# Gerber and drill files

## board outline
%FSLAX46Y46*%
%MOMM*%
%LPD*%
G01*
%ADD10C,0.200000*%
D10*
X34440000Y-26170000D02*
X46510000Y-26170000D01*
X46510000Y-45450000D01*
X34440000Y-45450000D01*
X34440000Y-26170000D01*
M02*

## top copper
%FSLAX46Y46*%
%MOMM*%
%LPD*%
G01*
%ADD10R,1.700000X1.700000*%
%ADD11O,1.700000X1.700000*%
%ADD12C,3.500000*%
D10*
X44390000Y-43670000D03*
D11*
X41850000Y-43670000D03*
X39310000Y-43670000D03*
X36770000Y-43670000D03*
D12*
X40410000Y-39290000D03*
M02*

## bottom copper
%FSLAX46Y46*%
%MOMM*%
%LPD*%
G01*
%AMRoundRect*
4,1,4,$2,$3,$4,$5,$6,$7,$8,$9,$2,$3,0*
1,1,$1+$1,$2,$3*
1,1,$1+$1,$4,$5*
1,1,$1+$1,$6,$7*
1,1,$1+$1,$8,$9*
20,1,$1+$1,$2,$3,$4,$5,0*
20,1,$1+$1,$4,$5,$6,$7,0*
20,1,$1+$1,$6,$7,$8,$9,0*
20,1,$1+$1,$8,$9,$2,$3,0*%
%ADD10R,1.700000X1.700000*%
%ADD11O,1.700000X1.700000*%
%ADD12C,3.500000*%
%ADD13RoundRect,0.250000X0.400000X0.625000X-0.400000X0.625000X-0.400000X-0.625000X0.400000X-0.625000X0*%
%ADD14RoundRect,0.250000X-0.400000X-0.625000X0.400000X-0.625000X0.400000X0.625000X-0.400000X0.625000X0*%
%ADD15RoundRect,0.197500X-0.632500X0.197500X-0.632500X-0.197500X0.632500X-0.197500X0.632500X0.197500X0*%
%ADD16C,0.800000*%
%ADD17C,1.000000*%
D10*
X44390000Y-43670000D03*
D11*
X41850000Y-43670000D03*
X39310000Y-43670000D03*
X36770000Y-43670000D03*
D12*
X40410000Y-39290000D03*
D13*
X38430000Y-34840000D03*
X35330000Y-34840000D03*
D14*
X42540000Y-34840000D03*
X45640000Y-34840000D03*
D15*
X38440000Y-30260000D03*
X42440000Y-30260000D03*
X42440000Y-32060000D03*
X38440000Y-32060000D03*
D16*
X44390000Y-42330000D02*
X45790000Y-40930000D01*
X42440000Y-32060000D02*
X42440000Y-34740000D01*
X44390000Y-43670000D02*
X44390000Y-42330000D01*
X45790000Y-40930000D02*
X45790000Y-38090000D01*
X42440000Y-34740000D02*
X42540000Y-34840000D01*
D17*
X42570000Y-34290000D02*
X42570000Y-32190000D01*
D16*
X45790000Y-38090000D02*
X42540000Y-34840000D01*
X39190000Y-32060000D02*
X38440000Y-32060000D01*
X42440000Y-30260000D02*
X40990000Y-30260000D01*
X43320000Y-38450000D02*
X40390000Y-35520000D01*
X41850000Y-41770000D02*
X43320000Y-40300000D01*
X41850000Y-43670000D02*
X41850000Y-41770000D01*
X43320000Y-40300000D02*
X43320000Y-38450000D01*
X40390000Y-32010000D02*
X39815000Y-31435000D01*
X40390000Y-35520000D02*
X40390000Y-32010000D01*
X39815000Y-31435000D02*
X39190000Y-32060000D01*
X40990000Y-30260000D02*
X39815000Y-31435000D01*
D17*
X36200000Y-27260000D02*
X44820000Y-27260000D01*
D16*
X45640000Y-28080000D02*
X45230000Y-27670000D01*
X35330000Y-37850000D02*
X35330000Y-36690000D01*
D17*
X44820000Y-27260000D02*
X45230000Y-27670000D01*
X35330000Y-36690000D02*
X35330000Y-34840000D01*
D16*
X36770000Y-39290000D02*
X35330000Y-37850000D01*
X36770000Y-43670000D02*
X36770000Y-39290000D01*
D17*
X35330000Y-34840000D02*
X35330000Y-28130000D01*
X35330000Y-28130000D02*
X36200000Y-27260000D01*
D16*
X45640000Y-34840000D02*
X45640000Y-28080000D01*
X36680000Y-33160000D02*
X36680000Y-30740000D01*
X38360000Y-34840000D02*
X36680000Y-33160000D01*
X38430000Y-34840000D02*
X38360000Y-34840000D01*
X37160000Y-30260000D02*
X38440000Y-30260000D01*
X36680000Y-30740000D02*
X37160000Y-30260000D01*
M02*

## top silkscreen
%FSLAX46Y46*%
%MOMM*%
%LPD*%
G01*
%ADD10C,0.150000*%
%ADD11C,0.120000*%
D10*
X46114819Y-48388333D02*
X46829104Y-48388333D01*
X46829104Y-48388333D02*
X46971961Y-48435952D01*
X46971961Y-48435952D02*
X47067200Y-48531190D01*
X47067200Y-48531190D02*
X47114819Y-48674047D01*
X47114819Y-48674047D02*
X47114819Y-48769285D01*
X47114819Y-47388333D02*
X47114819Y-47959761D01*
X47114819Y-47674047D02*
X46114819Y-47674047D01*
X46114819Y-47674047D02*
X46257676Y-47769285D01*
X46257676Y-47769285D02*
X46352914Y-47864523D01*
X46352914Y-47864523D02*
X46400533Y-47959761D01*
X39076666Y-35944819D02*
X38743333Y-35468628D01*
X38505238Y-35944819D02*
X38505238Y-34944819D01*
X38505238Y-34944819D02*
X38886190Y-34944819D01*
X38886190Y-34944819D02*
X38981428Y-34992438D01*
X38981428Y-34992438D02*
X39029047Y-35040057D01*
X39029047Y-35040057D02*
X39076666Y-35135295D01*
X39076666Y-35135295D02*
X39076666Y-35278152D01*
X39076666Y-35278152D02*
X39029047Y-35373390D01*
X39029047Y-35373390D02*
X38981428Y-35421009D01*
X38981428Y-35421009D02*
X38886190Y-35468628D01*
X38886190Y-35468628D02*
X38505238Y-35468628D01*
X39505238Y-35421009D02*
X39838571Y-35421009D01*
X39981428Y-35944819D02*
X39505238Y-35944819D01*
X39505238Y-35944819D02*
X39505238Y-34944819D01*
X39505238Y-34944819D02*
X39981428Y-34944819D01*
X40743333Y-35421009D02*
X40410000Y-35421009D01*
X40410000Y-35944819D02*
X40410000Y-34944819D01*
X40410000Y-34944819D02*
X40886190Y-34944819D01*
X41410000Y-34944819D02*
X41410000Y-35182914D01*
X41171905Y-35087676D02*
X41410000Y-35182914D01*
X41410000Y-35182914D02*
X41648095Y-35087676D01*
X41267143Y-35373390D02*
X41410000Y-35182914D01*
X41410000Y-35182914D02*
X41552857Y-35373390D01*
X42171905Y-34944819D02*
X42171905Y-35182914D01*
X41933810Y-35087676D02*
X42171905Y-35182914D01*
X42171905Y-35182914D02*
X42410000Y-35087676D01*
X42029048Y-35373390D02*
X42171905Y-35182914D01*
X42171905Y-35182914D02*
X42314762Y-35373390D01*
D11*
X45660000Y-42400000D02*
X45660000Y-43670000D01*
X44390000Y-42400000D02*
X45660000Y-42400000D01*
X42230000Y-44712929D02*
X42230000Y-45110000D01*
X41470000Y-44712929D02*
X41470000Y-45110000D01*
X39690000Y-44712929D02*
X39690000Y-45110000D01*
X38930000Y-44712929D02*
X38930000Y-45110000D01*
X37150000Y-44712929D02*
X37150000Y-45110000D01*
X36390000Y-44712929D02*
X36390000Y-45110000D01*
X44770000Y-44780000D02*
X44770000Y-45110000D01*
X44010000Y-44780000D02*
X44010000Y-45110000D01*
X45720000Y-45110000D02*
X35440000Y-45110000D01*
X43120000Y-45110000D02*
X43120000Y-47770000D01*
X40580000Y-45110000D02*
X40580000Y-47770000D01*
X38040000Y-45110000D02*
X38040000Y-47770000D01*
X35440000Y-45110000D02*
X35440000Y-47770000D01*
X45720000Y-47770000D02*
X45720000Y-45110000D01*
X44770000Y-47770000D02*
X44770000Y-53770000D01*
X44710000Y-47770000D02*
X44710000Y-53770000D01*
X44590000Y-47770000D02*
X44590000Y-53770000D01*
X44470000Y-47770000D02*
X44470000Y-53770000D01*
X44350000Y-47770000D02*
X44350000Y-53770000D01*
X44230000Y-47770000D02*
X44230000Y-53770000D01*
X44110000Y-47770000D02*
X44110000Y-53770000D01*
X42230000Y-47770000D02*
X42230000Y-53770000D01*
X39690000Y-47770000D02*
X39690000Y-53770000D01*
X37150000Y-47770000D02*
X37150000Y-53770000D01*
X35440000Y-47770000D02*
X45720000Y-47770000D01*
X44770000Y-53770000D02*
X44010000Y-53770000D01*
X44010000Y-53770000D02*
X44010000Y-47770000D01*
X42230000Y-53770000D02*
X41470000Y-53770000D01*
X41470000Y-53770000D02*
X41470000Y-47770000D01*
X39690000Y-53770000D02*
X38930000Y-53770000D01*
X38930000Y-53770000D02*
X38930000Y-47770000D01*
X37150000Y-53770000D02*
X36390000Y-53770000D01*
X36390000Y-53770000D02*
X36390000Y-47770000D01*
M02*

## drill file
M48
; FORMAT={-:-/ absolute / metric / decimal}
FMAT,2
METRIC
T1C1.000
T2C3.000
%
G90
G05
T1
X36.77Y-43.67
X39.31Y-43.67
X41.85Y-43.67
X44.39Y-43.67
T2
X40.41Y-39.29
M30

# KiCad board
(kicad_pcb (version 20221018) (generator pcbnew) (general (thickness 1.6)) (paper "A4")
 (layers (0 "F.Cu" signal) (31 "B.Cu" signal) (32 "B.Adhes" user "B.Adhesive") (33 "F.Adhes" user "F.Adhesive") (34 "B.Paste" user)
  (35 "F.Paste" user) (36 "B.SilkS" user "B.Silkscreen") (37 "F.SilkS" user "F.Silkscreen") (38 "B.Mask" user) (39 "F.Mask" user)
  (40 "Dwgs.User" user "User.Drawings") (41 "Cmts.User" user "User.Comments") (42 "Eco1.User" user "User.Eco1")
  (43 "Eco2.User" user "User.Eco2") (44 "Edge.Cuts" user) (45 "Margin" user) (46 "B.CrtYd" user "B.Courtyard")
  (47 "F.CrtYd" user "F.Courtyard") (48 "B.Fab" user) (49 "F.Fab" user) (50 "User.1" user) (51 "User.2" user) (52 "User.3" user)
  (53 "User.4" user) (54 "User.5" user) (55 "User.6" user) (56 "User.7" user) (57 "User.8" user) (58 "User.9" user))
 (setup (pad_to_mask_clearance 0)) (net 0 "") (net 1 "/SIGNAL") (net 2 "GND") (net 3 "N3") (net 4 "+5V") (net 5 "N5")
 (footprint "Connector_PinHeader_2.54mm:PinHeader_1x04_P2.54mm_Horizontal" (layer "F.Cu") (at 44.39 43.67 -90)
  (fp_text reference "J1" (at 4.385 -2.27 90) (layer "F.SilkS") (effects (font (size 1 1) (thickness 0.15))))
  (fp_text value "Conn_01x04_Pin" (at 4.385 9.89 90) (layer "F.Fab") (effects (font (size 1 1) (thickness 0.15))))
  (fp_line (start -1.27 -1.27) (end 0 -1.27) (stroke (width 0.12) (type solid)) (layer "F.SilkS"))
  (fp_line (start -1.27 0) (end -1.27 -1.27) (stroke (width 0.12) (type solid)) (layer "F.SilkS"))
  (fp_line (start 1.042929 2.16) (end 1.44 2.16) (stroke (width 0.12) (type solid)) (layer "F.SilkS"))
  (fp_line (start 1.042929 2.92) (end 1.44 2.92) (stroke (width 0.12) (type solid)) (layer "F.SilkS"))
  (fp_line (start 1.042929 4.7) (end 1.44 4.7) (stroke (width 0.12) (type solid)) (layer "F.SilkS"))
  (fp_line (start 1.042929 5.46) (end 1.44 5.46) (stroke (width 0.12) (type solid)) (layer "F.SilkS"))
  (fp_line (start 1.042929 7.24) (end 1.44 7.24) (stroke (width 0.12) (type solid)) (layer "F.SilkS"))
  (fp_line (start 1.042929 8) (end 1.44 8) (stroke (width 0.12) (type solid)) (layer "F.SilkS"))
  (fp_line (start 1.11 -0.38) (end 1.44 -0.38) (stroke (width 0.12) (type solid)) (layer "F.SilkS"))
  (fp_line (start 1.11 0.38) (end 1.44 0.38) (stroke (width 0.12) (type solid)) (layer "F.SilkS"))
  (fp_line (start 1.44 -1.33) (end 1.44 8.95) (stroke (width 0.12) (type solid)) (layer "F.SilkS"))
  (fp_line (start 1.44 1.27) (end 4.1 1.27) (stroke (width 0.12) (type solid)) (layer "F.SilkS"))
  (fp_line (start 1.44 3.81) (end 4.1 3.81) (stroke (width 0.12) (type solid)) (layer "F.SilkS"))
  (fp_line (start 1.44 6.35) (end 4.1 6.35) (stroke (width 0.12) (type solid)) (layer "F.SilkS"))
  (fp_line (start 1.44 8.95) (end 4.1 8.95) (stroke (width 0.12) (type solid)) (layer "F.SilkS"))
  (fp_line (start 4.1 -1.33) (end 1.44 -1.33) (stroke (width 0.12) (type solid)) (layer "F.SilkS"))
  (fp_line (start 4.1 -0.38) (end 10.1 -0.38) (stroke (width 0.12) (type solid)) (layer "F.SilkS"))
  (fp_line (start 4.1 -0.32) (end 10.1 -0.32) (stroke (width 0.12) (type solid)) (layer "F.SilkS"))
  (fp_line (start 4.1 -0.2) (end 10.1 -0.2) (stroke (width 0.12) (type solid)) (layer "F.SilkS"))
  (fp_line (start 4.1 -0.08) (end 10.1 -0.08) (stroke (width 0.12) (type solid)) (layer "F.SilkS"))
  (fp_line (start 4.1 0.04) (end 10.1 0.04) (stroke (width 0.12) (type solid)) (layer "F.SilkS"))
  (fp_line (start 4.1 0.16) (end 10.1 0.16) (stroke (width 0.12) (type solid)) (layer "F.SilkS"))
  (fp_line (start 4.1 0.28) (end 10.1 0.28) (stroke (width 0.12) (type solid)) (layer "F.SilkS"))
  (fp_line (start 4.1 2.16) (end 10.1 2.16) (stroke (width 0.12) (type solid)) (layer "F.SilkS"))
  (fp_line (start 4.1 4.7) (end 10.1 4.7) (stroke (width 0.12) (type solid)) (layer "F.SilkS"))
  (fp_line (start 4.1 7.24) (end 10.1 7.24) (stroke (width 0.12) (type solid)) (layer "F.SilkS"))
  (fp_line (start 4.1 8.95) (end 4.1 -1.33) (stroke (width 0.12) (type solid)) (layer "F.SilkS"))
  (fp_line (start 10.1 -0.38) (end 10.1 0.38) (stroke (width 0.12) (type solid)) (layer "F.SilkS"))
  (fp_line (start 10.1 0.38) (end 4.1 0.38) (stroke (width 0.12) (type solid)) (layer "F.SilkS"))
  (fp_line (start 10.1 2.16) (end 10.1 2.92) (stroke (width 0.12) (type solid)) (layer "F.SilkS"))
  (fp_line (start 10.1 2.92) (end 4.1 2.92) (stroke (width 0.12) (type solid)) (layer "F.SilkS"))
  (fp_line (start 10.1 4.7) (end 10.1 5.46) (stroke (width 0.12) (type solid)) (layer "F.SilkS"))
  (fp_line (start 10.1 5.46) (end 4.1 5.46) (stroke (width 0.12) (type solid)) (layer "F.SilkS"))
  (fp_line (start 10.1 7.24) (end 10.1 8) (stroke (width 0.12) (type solid)) (layer "F.SilkS"))
  (fp_line (start 10.1 8) (end 4.1 8) (stroke (width 0.12) (type solid)) (layer "F.SilkS"))
  (pad "1" thru_hole rect (at 0 0 270) (size 1.7 1.7) (drill 1) (layers "*.Cu" "*.Mask") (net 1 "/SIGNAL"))
  (pad "2" thru_hole oval (at 0 2.54 270) (size 1.7 1.7) (drill 1) (layers "*.Cu" "*.Mask") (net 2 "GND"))
  (pad "3" thru_hole oval (at 0 5.08 270) (size 1.7 1.7) (drill 1) (layers "*.Cu" "*.Mask") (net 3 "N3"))
  (pad "4" thru_hole oval (at 0 7.62 270) (size 1.7 1.7) (drill 1) (layers "*.Cu" "*.Mask") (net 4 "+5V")))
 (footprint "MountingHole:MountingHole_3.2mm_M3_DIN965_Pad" (layer "F.Cu") (at 40.41 39.29)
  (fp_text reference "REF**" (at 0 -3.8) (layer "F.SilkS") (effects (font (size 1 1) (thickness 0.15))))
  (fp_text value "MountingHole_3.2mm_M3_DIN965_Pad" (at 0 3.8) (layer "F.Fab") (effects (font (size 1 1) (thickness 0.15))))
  (pad "1" thru_hole circle (at 0 0) (size 3.5 3.5) (drill 3) (layers "*.Cu" "*.Mask")))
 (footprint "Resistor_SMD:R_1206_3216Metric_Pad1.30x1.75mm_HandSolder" (layer "B.Cu") (at 36.88 34.84 180)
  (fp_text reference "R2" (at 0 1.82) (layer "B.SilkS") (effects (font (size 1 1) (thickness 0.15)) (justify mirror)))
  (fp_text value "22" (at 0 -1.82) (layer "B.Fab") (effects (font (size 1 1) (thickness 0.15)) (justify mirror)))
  (pad "1" smd roundrect (at -1.55 0 180) (size 1.3 1.75) (layers "B.Cu" "B.Paste" "B.Mask") (roundrect_rratio 0.192308) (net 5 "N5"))
  (pad "2" smd roundrect (at 1.55 0 180) (size 1.3 1.75) (layers "B.Cu" "B.Paste" "B.Mask") (roundrect_rratio 0.192308) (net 4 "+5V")))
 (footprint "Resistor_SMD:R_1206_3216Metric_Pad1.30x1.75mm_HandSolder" (layer "B.Cu") (at 44.09 34.84)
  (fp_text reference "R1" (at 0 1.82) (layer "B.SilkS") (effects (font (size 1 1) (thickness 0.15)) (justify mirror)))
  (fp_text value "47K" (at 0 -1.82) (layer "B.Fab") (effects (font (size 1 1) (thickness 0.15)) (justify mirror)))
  (pad "1" smd roundrect (at -1.55 0) (size 1.3 1.75) (layers "B.Cu" "B.Paste" "B.Mask") (roundrect_rratio 0.192308) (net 1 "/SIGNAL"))
  (pad "2" smd roundrect (at 1.55 0) (size 1.3 1.75) (layers "B.Cu" "B.Paste" "B.Mask") (roundrect_rratio 0.192308) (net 4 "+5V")))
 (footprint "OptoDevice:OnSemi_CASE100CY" (layer "B.Cu") (at 40.44 31.16 -90)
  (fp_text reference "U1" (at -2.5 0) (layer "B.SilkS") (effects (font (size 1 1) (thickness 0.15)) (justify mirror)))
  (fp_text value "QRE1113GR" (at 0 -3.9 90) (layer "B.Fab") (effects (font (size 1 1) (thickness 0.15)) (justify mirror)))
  (pad "1" smd roundrect (at -0.9 2 270) (size 0.79 1.66) (layers "B.Cu" "B.Paste" "B.Mask") (roundrect_rratio 0.25) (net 5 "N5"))
  (pad "2" smd roundrect (at -0.9 -2 270) (size 0.79 1.66) (layers "B.Cu" "B.Paste" "B.Mask") (roundrect_rratio 0.25) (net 2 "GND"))
  (pad "3" smd roundrect (at 0.9 -2 270) (size 0.79 1.66) (layers "B.Cu" "B.Paste" "B.Mask") (roundrect_rratio 0.25) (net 1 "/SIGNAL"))
  (pad "4" smd roundrect (at 0.9 2 270) (size 0.79 1.66) (layers "B.Cu" "B.Paste" "B.Mask") (roundrect_rratio 0.25) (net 2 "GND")))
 (gr_rect (start 34.44 26.17) (end 46.51 45.45) (stroke (width 0.2) (type default)) (fill none) (layer "Edge.Cuts"))
 (segment (start 44.39 42.33) (end 45.79 40.93) (width 0.8) (layer "B.Cu") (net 1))
 (segment (start 42.44 32.06) (end 42.44 34.74) (width 0.8) (layer "B.Cu") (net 1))
 (segment (start 44.39 43.67) (end 44.39 42.33) (width 0.8) (layer "B.Cu") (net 1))
 (segment (start 45.79 40.93) (end 45.79 38.09) (width 0.8) (layer "B.Cu") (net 1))
 (segment (start 42.44 34.74) (end 42.54 34.84) (width 0.8) (layer "B.Cu") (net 1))
 (segment (start 42.57 34.29) (end 42.57 32.19) (width 1) (layer "B.Cu") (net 1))
 (segment (start 45.79 38.09) (end 42.54 34.84) (width 0.8) (layer "B.Cu") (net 1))
 (segment (start 39.19 32.06) (end 38.44 32.06) (width 0.8) (layer "B.Cu") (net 2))
 (segment (start 42.44 30.26) (end 40.99 30.26) (width 0.8) (layer "B.Cu") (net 2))
 (segment (start 43.32 38.45) (end 40.39 35.52) (width 0.8) (layer "B.Cu") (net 2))
 (segment (start 41.85 41.77) (end 43.32 40.3) (width 0.8) (layer "B.Cu") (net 2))
 (segment (start 41.85 43.67) (end 41.85 41.77) (width 0.8) (layer "B.Cu") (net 2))
 (segment (start 43.32 40.3) (end 43.32 38.45) (width 0.8) (layer "B.Cu") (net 2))
 (segment (start 40.39 32.01) (end 39.815 31.435) (width 0.8) (layer "B.Cu") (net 2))
 (segment (start 40.39 35.52) (end 40.39 32.01) (width 0.8) (layer "B.Cu") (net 2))
 (segment (start 39.815 31.435) (end 39.19 32.06) (width 0.8) (layer "B.Cu") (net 2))
 (segment (start 40.99 30.26) (end 39.815 31.435) (width 0.8) (layer "B.Cu") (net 2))
 (segment (start 36.2 27.26) (end 44.82 27.26) (width 1) (layer "B.Cu") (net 4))
 (segment (start 45.64 28.08) (end 45.23 27.67) (width 0.8) (layer "B.Cu") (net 4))
 (segment (start 35.33 37.85) (end 35.33 36.69) (width 0.8) (layer "B.Cu") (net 4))
 (segment (start 44.82 27.26) (end 45.23 27.67) (width 1) (layer "B.Cu") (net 4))
 (segment (start 35.33 36.69) (end 35.33 34.84) (width 1) (layer "B.Cu") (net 4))
 (segment (start 36.77 39.29) (end 35.33 37.85) (width 0.8) (layer "B.Cu") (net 4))
 (segment (start 36.77 43.67) (end 36.77 39.29) (width 0.8) (layer "B.Cu") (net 4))
 (segment (start 35.33 34.84) (end 35.33 28.13) (width 1) (layer "B.Cu") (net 4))
 (segment (start 35.33 28.13) (end 36.2 27.26) (width 1) (layer "B.Cu") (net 4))
 (segment (start 45.64 34.84) (end 45.64 28.08) (width 0.8) (layer "B.Cu") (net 4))
 (segment (start 36.68 33.16) (end 36.68 30.74) (width 0.8) (layer "B.Cu") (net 5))
 (segment (start 38.36 34.84) (end 36.68 33.16) (width 0.8) (layer "B.Cu") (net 5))
 (segment (start 38.43 34.84) (end 38.36 34.84) (width 0.8) (layer "B.Cu") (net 5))
 (segment (start 37.16 30.26) (end 38.44 30.26) (width 0.8) (layer "B.Cu") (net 5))
 (segment (start 36.68 30.74) (end 37.16 30.26) (width 0.8) (layer "B.Cu") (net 5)))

